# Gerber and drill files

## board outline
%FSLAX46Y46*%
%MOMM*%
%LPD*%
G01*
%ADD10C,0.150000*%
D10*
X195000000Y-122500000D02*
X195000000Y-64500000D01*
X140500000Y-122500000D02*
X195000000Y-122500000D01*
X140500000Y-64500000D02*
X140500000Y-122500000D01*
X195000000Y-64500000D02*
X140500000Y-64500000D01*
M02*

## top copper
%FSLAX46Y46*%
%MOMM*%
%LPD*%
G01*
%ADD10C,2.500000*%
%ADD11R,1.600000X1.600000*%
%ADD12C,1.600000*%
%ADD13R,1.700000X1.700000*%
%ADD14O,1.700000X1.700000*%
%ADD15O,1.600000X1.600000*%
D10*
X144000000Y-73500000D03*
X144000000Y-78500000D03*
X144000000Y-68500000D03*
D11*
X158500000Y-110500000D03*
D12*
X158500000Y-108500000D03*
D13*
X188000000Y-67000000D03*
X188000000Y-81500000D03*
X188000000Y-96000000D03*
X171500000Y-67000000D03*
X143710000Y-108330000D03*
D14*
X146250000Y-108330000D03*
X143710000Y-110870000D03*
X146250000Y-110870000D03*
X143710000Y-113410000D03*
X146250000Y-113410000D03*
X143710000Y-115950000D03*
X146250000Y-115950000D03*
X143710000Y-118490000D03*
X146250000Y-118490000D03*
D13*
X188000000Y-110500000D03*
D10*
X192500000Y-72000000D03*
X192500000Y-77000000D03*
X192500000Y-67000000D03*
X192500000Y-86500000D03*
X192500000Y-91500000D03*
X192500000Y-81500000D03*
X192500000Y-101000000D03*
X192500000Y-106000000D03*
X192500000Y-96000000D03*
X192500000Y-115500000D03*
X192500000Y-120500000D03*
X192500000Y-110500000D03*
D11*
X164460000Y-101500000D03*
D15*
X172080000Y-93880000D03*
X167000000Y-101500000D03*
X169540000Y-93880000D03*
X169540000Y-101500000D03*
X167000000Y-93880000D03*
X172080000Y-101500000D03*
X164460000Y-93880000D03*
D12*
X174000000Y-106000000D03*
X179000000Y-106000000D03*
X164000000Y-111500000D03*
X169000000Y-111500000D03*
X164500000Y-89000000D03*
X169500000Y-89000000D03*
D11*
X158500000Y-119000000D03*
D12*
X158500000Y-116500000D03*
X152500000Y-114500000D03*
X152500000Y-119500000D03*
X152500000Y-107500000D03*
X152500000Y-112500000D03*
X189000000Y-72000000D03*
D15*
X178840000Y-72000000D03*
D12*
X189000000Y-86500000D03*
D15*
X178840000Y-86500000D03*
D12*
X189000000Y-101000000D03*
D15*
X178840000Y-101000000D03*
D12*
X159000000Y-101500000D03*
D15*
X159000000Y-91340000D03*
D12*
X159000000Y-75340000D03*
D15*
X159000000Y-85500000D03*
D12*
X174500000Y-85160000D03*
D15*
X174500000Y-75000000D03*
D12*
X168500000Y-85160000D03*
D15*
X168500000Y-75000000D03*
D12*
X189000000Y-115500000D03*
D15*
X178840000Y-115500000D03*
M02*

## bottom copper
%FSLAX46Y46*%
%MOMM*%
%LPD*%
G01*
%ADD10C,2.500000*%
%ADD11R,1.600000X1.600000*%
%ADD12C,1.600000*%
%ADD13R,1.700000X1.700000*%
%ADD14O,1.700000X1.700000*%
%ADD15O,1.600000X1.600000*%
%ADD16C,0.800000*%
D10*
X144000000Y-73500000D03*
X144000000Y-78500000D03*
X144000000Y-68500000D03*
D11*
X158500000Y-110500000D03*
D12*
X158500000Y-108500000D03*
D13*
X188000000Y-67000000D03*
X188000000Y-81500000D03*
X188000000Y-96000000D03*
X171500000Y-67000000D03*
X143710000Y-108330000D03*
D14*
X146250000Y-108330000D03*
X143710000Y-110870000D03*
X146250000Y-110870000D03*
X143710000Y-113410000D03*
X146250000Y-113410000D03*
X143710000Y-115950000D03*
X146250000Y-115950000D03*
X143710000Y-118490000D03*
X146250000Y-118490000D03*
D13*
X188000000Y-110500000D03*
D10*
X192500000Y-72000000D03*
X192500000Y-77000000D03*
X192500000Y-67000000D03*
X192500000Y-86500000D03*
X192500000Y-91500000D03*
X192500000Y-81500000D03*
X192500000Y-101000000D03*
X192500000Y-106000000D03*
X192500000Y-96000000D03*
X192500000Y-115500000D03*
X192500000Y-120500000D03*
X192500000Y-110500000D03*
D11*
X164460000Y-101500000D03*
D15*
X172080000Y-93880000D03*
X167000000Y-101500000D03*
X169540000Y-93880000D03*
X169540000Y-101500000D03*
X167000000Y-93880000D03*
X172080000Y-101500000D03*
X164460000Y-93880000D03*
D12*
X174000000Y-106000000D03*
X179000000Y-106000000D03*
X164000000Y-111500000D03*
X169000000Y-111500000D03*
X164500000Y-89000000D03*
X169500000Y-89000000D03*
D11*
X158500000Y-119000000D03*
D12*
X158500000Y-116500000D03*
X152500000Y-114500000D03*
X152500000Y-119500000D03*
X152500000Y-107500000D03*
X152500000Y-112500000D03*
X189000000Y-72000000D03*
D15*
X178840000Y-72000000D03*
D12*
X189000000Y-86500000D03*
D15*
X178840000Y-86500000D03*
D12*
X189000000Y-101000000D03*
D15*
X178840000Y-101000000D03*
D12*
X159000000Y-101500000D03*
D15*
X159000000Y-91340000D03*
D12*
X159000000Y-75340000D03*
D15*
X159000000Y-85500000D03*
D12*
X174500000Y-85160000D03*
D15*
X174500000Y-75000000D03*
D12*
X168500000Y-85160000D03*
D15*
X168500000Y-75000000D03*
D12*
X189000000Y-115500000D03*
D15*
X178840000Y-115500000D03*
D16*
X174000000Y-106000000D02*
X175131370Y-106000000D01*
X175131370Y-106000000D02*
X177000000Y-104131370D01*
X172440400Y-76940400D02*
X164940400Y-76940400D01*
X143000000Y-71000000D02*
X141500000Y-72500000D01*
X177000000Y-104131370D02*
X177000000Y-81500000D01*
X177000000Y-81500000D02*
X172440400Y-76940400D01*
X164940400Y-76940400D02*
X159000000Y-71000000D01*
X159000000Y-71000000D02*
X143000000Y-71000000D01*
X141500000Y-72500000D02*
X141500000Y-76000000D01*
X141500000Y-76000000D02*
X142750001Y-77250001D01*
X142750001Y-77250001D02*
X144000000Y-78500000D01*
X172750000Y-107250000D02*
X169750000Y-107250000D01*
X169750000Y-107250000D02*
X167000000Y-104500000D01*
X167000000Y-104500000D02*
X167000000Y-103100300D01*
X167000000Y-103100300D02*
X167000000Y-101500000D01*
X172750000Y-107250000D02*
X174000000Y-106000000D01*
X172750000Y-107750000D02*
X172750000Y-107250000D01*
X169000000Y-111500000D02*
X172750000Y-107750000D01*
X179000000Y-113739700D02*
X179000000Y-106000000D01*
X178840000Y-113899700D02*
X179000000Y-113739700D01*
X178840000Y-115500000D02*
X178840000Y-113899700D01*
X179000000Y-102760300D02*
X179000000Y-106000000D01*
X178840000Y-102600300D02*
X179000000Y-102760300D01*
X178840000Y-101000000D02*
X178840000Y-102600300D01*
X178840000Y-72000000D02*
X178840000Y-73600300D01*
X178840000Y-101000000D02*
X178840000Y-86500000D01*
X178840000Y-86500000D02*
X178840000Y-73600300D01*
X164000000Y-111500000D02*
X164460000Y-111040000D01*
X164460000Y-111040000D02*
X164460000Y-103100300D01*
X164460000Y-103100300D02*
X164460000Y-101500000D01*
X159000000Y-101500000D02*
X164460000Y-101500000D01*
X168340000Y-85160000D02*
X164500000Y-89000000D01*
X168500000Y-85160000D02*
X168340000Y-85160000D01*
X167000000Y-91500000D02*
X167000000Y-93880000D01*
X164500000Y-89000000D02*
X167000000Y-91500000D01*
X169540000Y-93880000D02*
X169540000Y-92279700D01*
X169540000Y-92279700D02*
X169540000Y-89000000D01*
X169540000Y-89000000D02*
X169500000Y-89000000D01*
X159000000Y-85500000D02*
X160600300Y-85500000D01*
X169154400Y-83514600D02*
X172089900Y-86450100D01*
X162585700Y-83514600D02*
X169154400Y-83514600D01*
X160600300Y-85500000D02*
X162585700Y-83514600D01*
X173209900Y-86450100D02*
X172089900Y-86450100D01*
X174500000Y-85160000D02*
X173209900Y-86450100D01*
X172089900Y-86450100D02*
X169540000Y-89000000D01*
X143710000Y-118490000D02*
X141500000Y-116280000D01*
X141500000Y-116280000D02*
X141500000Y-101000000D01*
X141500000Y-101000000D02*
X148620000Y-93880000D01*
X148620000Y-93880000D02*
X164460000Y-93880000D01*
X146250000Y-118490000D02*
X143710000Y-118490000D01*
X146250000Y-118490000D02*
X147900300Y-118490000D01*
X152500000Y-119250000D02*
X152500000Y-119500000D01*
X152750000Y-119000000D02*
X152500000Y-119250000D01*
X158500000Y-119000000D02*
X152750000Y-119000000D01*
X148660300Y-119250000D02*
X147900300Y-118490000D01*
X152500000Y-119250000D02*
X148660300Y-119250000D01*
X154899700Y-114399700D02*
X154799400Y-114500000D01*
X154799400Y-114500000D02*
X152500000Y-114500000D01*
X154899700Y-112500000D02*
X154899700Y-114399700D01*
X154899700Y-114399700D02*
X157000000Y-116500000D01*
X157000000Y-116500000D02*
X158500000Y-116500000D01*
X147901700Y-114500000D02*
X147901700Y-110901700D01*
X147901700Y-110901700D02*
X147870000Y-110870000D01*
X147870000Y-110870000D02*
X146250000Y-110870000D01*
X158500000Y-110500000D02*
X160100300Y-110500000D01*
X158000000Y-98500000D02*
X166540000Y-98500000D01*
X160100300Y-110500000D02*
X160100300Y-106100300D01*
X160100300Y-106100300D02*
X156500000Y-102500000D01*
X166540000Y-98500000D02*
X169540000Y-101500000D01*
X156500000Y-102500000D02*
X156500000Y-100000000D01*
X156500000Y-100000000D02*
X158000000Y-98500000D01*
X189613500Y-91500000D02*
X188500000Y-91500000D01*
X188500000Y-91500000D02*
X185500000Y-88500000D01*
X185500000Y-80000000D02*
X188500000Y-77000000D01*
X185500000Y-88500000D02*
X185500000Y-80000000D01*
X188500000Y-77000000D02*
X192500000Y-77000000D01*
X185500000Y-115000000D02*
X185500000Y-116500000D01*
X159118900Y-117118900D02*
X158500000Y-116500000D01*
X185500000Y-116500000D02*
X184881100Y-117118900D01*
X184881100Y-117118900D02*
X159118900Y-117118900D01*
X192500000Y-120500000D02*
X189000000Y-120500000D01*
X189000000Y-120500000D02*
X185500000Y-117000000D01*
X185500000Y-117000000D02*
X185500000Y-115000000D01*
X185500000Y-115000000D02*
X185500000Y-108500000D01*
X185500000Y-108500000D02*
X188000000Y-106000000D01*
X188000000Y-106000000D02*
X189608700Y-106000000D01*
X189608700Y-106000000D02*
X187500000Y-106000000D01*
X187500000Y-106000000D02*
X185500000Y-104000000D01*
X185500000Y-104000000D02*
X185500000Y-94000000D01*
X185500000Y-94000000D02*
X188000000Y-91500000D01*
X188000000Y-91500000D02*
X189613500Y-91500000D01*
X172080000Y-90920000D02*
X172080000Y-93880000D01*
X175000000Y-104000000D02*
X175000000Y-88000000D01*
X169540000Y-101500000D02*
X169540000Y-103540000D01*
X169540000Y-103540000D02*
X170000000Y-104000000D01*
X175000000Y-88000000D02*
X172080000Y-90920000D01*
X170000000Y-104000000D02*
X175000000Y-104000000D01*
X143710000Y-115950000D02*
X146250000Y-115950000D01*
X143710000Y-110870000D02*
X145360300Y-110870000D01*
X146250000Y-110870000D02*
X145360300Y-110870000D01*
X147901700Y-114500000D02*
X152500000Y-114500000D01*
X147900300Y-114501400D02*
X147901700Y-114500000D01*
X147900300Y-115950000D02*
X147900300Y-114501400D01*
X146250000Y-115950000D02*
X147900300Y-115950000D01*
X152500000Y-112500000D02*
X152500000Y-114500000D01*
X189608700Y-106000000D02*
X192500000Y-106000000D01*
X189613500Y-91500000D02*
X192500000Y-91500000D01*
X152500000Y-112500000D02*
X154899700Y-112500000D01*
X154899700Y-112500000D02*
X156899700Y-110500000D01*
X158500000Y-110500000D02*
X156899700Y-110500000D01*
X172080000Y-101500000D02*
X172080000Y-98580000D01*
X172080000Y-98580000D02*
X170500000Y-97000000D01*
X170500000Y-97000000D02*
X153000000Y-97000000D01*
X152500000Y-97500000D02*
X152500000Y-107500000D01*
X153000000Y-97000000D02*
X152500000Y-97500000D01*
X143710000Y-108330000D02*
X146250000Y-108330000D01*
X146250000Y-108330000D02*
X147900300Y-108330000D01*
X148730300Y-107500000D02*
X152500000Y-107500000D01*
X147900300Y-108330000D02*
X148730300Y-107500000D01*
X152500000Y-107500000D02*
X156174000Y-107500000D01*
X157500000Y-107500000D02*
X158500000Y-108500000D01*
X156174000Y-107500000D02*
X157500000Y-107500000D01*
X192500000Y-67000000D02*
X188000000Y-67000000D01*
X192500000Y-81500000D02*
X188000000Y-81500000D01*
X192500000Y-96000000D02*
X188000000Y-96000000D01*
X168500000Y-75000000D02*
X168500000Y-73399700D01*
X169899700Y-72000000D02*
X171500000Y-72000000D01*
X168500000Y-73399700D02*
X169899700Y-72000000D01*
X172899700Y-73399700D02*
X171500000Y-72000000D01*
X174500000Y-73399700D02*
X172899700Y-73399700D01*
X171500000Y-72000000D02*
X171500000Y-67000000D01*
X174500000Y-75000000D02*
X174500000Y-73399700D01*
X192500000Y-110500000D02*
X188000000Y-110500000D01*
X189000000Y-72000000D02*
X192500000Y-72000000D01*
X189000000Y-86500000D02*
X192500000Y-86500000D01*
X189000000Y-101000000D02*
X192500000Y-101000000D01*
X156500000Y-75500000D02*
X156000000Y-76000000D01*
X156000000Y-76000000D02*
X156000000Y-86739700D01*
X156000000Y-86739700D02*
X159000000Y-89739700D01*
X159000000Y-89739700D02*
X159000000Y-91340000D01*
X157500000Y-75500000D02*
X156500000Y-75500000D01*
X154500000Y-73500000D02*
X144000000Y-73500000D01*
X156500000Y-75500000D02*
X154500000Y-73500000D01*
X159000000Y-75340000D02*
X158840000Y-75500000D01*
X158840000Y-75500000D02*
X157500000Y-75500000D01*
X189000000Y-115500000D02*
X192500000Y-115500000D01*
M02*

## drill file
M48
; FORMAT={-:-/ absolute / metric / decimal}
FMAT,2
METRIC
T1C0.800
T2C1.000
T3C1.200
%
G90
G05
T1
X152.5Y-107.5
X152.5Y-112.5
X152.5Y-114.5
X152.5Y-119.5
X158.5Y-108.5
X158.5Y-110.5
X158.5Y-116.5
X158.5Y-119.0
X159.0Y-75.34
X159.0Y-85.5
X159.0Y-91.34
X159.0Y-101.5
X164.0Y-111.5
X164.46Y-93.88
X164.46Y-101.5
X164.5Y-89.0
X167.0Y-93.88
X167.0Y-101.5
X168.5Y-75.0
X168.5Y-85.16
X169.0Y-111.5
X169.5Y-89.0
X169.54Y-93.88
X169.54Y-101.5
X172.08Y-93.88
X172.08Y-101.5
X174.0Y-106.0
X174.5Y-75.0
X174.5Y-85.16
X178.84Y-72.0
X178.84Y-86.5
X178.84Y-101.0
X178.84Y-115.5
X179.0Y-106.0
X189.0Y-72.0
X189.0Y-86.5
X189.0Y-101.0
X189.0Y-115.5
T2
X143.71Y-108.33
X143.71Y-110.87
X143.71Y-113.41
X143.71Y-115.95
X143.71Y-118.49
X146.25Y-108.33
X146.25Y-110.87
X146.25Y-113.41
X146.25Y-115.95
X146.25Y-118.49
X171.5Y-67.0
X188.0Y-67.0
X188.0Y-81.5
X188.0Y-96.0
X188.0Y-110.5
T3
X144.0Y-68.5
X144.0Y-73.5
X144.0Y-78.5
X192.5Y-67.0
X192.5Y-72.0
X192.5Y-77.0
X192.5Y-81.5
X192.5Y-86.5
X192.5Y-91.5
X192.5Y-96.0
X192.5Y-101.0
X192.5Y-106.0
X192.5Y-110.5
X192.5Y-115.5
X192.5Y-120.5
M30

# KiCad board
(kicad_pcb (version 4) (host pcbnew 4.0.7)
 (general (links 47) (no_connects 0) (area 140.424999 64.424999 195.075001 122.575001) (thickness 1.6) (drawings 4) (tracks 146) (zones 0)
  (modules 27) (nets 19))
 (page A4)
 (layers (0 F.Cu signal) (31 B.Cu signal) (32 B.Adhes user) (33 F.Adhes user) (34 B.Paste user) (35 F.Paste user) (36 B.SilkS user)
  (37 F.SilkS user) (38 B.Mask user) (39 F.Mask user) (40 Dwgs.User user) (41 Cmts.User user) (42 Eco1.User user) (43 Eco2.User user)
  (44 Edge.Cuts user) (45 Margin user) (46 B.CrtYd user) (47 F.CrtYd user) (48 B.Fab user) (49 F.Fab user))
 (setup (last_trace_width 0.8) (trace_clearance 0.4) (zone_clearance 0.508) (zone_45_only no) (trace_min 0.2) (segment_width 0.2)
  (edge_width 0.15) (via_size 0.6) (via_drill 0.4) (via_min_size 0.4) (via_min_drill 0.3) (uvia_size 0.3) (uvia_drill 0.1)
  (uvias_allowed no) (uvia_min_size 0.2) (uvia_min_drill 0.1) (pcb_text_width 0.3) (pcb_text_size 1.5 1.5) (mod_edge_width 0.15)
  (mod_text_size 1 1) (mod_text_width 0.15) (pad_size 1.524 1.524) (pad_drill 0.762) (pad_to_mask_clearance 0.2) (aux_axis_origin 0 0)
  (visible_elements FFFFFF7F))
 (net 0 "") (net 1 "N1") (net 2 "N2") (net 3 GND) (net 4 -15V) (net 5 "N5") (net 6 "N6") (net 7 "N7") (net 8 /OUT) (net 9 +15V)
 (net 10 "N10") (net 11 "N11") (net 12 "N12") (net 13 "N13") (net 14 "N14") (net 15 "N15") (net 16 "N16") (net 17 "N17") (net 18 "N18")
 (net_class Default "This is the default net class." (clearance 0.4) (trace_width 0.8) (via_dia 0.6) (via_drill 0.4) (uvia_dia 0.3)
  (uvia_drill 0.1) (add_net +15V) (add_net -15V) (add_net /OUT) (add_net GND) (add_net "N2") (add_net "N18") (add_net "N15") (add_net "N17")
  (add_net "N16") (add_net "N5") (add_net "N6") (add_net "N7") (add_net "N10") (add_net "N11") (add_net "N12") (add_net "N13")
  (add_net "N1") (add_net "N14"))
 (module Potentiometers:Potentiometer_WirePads (layer F.Cu) (at 144 68.5)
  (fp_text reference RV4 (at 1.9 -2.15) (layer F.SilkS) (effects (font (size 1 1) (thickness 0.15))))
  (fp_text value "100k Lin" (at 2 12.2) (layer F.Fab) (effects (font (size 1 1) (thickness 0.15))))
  (pad 2 thru_hole circle (at 0 5) (size 2.5 2.5) (drill 1.2) (layers *.Cu *.Mask) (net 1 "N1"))
  (pad 3 thru_hole circle (at 0 10) (size 2.5 2.5) (drill 1.2) (layers *.Cu *.Mask) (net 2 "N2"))
  (pad 1 thru_hole circle (at 0 0) (size 2.5 2.5) (drill 1.2) (layers *.Cu *.Mask)))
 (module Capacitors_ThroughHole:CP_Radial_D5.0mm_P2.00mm (layer F.Cu) (at 158.5 110.5 90)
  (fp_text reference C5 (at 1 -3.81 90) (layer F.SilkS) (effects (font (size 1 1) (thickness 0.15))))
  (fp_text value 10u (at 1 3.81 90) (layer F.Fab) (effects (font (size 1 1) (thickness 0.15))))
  (pad 1 thru_hole rect (at 0 0 90) (size 1.6 1.6) (drill 0.8) (layers *.Cu *.Mask) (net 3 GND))
  (pad 2 thru_hole circle (at 2 0 90) (size 1.6 1.6) (drill 0.8) (layers *.Cu *.Mask) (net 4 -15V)))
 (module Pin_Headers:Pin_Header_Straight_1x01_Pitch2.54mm (layer F.Cu) (at 188 67)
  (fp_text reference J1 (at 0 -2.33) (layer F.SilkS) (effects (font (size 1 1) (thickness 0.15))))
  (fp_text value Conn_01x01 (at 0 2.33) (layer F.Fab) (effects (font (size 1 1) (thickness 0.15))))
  (pad 1 thru_hole rect (at 0 0) (size 1.7 1.7) (drill 1) (layers *.Cu *.Mask) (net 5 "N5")))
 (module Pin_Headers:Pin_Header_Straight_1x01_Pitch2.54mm (layer F.Cu) (at 188 81.5)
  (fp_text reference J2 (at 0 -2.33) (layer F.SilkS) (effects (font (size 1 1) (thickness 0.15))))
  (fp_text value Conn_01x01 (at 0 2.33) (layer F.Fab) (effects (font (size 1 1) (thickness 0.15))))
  (pad 1 thru_hole rect (at 0 0) (size 1.7 1.7) (drill 1) (layers *.Cu *.Mask) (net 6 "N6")))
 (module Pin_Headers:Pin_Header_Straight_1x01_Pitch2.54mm (layer F.Cu) (at 188 96)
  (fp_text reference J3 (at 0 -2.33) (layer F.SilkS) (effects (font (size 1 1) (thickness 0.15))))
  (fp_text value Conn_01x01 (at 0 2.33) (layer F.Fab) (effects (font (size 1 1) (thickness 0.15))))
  (pad 1 thru_hole rect (at 0 0) (size 1.7 1.7) (drill 1) (layers *.Cu *.Mask) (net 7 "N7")))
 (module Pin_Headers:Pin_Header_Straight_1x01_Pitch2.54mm (layer F.Cu) (at 171.5 67)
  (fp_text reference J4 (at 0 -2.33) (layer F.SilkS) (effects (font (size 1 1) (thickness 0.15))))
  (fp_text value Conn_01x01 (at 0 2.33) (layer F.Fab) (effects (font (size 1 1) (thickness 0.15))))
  (pad 1 thru_hole rect (at 0 0) (size 1.7 1.7) (drill 1) (layers *.Cu *.Mask) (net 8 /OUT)))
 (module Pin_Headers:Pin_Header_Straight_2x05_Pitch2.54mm (layer F.Cu) (at 143.71 108.33)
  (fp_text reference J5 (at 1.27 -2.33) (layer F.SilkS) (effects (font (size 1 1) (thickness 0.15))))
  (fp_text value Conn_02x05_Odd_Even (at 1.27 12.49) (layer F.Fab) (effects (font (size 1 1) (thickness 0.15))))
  (pad 1 thru_hole rect (at 0 0) (size 1.7 1.7) (drill 1) (layers *.Cu *.Mask) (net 4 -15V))
  (pad 2 thru_hole oval (at 2.54 0) (size 1.7 1.7) (drill 1) (layers *.Cu *.Mask) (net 4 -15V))
  (pad 3 thru_hole oval (at 0 2.54) (size 1.7 1.7) (drill 1) (layers *.Cu *.Mask) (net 3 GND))
  (pad 4 thru_hole oval (at 2.54 2.54) (size 1.7 1.7) (drill 1) (layers *.Cu *.Mask) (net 3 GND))
  (pad 5 thru_hole oval (at 0 5.08) (size 1.7 1.7) (drill 1) (layers *.Cu *.Mask))
  (pad 6 thru_hole oval (at 2.54 5.08) (size 1.7 1.7) (drill 1) (layers *.Cu *.Mask))
  (pad 7 thru_hole oval (at 0 7.62) (size 1.7 1.7) (drill 1) (layers *.Cu *.Mask) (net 3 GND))
  (pad 8 thru_hole oval (at 2.54 7.62) (size 1.7 1.7) (drill 1) (layers *.Cu *.Mask) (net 3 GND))
  (pad 9 thru_hole oval (at 0 10.16) (size 1.7 1.7) (drill 1) (layers *.Cu *.Mask) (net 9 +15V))
  (pad 10 thru_hole oval (at 2.54 10.16) (size 1.7 1.7) (drill 1) (layers *.Cu *.Mask) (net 9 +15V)))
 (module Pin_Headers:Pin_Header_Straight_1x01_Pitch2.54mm (layer F.Cu) (at 188 110.5)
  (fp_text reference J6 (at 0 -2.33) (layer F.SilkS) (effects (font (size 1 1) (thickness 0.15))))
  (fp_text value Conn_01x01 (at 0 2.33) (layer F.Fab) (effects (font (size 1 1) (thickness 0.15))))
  (pad 1 thru_hole rect (at 0 0) (size 1.7 1.7) (drill 1) (layers *.Cu *.Mask) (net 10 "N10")))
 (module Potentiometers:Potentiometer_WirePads (layer F.Cu) (at 192.5 67)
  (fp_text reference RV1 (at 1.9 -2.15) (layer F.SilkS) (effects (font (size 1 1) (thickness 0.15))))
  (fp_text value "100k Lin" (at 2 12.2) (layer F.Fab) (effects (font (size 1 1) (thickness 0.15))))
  (pad 2 thru_hole circle (at 0 5) (size 2.5 2.5) (drill 1.2) (layers *.Cu *.Mask) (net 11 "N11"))
  (pad 3 thru_hole circle (at 0 10) (size 2.5 2.5) (drill 1.2) (layers *.Cu *.Mask) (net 3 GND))
  (pad 1 thru_hole circle (at 0 0) (size 2.5 2.5) (drill 1.2) (layers *.Cu *.Mask) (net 5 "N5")))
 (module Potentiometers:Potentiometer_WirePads (layer F.Cu) (at 192.5 81.5)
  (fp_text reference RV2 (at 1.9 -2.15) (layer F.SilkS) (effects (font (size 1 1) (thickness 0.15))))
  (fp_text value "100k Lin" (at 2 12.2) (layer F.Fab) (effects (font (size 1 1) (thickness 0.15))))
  (pad 2 thru_hole circle (at 0 5) (size 2.5 2.5) (drill 1.2) (layers *.Cu *.Mask) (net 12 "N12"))
  (pad 3 thru_hole circle (at 0 10) (size 2.5 2.5) (drill 1.2) (layers *.Cu *.Mask) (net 3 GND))
  (pad 1 thru_hole circle (at 0 0) (size 2.5 2.5) (drill 1.2) (layers *.Cu *.Mask) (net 6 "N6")))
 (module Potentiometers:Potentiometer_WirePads (layer F.Cu) (at 192.5 96)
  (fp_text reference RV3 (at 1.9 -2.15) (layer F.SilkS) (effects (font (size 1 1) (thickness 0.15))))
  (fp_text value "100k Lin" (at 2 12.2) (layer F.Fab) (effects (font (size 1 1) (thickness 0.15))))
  (pad 2 thru_hole circle (at 0 5) (size 2.5 2.5) (drill 1.2) (layers *.Cu *.Mask) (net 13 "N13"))
  (pad 3 thru_hole circle (at 0 10) (size 2.5 2.5) (drill 1.2) (layers *.Cu *.Mask) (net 3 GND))
  (pad 1 thru_hole circle (at 0 0) (size 2.5 2.5) (drill 1.2) (layers *.Cu *.Mask) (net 7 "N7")))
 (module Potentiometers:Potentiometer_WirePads (layer F.Cu) (at 192.5 110.5)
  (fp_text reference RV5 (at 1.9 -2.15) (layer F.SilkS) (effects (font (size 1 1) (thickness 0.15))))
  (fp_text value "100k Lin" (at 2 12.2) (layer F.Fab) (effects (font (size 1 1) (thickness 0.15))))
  (pad 2 thru_hole circle (at 0 5) (size 2.5 2.5) (drill 1.2) (layers *.Cu *.Mask) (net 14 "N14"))
  (pad 3 thru_hole circle (at 0 10) (size 2.5 2.5) (drill 1.2) (layers *.Cu *.Mask) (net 3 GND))
  (pad 1 thru_hole circle (at 0 0) (size 2.5 2.5) (drill 1.2) (layers *.Cu *.Mask) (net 10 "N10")))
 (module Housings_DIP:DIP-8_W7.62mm (layer F.Cu) (at 164.46 101.5 90)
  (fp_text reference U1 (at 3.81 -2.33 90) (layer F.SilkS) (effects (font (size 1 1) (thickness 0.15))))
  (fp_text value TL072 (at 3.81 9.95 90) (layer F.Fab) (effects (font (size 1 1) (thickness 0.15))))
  (pad 1 thru_hole rect (at 0 0 90) (size 1.6 1.6) (drill 0.8) (layers *.Cu *.Mask) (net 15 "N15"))
  (pad 5 thru_hole oval (at 7.62 7.62 90) (size 1.6 1.6) (drill 0.8) (layers *.Cu *.Mask) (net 3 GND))
  (pad 2 thru_hole oval (at 0 2.54 90) (size 1.6 1.6) (drill 0.8) (layers *.Cu *.Mask) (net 2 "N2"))
  (pad 6 thru_hole oval (at 7.62 5.08 90) (size 1.6 1.6) (drill 0.8) (layers *.Cu *.Mask) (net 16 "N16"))
  (pad 3 thru_hole oval (at 0 5.08 90) (size 1.6 1.6) (drill 0.8) (layers *.Cu *.Mask) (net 3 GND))
  (pad 7 thru_hole oval (at 7.62 2.54 90) (size 1.6 1.6) (drill 0.8) (layers *.Cu *.Mask) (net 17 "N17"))
  (pad 4 thru_hole oval (at 0 7.62 90) (size 1.6 1.6) (drill 0.8) (layers *.Cu *.Mask) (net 4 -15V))
  (pad 8 thru_hole oval (at 7.62 0 90) (size 1.6 1.6) (drill 0.8) (layers *.Cu *.Mask) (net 9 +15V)))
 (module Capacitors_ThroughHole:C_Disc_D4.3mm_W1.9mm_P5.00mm (layer F.Cu) (at 174 106)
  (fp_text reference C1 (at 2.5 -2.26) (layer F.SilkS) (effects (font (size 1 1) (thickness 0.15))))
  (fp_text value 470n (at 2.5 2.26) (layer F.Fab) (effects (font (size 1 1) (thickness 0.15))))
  (pad 1 thru_hole circle (at 0 0) (size 1.6 1.6) (drill 0.8) (layers *.Cu *.Mask) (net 2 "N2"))
  (pad 2 thru_hole circle (at 5 0) (size 1.6 1.6) (drill 0.8) (layers *.Cu *.Mask) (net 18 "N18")))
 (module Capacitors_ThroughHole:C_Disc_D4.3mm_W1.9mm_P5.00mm (layer F.Cu) (at 164 111.5)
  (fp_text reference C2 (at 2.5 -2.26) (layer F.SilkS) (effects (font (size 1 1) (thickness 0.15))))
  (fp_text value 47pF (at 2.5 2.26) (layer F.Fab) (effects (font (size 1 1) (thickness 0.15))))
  (pad 1 thru_hole circle (at 0 0) (size 1.6 1.6) (drill 0.8) (layers *.Cu *.Mask) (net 15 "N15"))
  (pad 2 thru_hole circle (at 5 0) (size 1.6 1.6) (drill 0.8) (layers *.Cu *.Mask) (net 2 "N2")))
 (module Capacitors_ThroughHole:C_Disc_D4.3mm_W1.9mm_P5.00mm (layer F.Cu) (at 164.5 89)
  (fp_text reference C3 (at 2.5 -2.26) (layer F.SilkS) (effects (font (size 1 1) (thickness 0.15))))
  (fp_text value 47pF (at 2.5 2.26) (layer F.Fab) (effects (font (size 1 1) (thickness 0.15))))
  (pad 1 thru_hole circle (at 0 0) (size 1.6 1.6) (drill 0.8) (layers *.Cu *.Mask) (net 17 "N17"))
  (pad 2 thru_hole circle (at 5 0) (size 1.6 1.6) (drill 0.8) (layers *.Cu *.Mask) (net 16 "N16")))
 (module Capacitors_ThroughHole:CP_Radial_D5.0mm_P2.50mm (layer F.Cu) (at 158.5 119 90)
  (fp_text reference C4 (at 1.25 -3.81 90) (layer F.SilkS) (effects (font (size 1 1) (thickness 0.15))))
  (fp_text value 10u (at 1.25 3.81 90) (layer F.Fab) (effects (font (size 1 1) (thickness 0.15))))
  (pad 1 thru_hole rect (at 0 0 90) (size 1.6 1.6) (drill 0.8) (layers *.Cu *.Mask) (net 9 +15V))
  (pad 2 thru_hole circle (at 2.5 0 90) (size 1.6 1.6) (drill 0.8) (layers *.Cu *.Mask) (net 3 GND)))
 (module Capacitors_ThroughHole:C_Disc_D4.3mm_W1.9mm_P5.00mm (layer F.Cu) (at 152.5 114.5 270)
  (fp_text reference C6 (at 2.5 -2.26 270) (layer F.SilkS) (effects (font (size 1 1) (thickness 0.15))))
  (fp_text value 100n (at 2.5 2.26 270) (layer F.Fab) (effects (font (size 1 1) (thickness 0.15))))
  (pad 1 thru_hole circle (at 0 0 270) (size 1.6 1.6) (drill 0.8) (layers *.Cu *.Mask) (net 3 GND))
  (pad 2 thru_hole circle (at 5 0 270) (size 1.6 1.6) (drill 0.8) (layers *.Cu *.Mask) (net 9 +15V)))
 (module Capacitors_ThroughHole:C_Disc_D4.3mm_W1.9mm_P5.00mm (layer F.Cu) (at 152.5 107.5 270)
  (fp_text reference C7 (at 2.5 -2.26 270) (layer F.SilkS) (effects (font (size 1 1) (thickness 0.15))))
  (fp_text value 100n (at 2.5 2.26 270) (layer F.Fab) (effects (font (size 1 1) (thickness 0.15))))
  (pad 1 thru_hole circle (at 0 0 270) (size 1.6 1.6) (drill 0.8) (layers *.Cu *.Mask) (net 4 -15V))
  (pad 2 thru_hole circle (at 5 0 270) (size 1.6 1.6) (drill 0.8) (layers *.Cu *.Mask) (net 3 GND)))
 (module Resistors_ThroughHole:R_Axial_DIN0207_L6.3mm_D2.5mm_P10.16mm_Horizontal (layer F.Cu) (at 189 72 180)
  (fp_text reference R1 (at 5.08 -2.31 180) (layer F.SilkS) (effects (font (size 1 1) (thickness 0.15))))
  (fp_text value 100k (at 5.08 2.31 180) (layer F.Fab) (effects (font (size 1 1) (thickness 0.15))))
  (pad 1 thru_hole circle (at 0 0 180) (size 1.6 1.6) (drill 0.8) (layers *.Cu *.Mask) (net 11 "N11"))
  (pad 2 thru_hole oval (at 10.16 0 180) (size 1.6 1.6) (drill 0.8) (layers *.Cu *.Mask) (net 18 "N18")))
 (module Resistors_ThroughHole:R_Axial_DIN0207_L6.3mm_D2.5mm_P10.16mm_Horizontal (layer F.Cu) (at 189 86.5 180)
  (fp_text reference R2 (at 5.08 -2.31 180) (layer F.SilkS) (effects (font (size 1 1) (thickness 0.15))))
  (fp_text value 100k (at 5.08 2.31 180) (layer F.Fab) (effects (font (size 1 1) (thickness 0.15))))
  (pad 1 thru_hole circle (at 0 0 180) (size 1.6 1.6) (drill 0.8) (layers *.Cu *.Mask) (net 12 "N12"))
  (pad 2 thru_hole oval (at 10.16 0 180) (size 1.6 1.6) (drill 0.8) (layers *.Cu *.Mask) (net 18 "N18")))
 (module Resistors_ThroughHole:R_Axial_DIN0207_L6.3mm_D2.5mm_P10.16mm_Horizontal (layer F.Cu) (at 189 101 180)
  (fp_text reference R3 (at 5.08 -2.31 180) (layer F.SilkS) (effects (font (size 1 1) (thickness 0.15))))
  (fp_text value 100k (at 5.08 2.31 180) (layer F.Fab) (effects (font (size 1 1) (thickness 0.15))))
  (pad 1 thru_hole circle (at 0 0 180) (size 1.6 1.6) (drill 0.8) (layers *.Cu *.Mask) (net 13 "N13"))
  (pad 2 thru_hole oval (at 10.16 0 180) (size 1.6 1.6) (drill 0.8) (layers *.Cu *.Mask) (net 18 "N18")))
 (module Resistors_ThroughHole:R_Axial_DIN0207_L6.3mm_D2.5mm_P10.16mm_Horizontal (layer F.Cu) (at 159 101.5 90)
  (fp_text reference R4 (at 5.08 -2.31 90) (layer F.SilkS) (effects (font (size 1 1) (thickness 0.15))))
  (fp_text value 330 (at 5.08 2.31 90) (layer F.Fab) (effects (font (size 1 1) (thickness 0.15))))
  (pad 1 thru_hole circle (at 0 0 90) (size 1.6 1.6) (drill 0.8) (layers *.Cu *.Mask) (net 15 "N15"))
  (pad 2 thru_hole oval (at 10.16 0 90) (size 1.6 1.6) (drill 0.8) (layers *.Cu *.Mask) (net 1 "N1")))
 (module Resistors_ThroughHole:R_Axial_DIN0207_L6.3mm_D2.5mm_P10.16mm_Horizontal (layer F.Cu) (at 159 75.34 270)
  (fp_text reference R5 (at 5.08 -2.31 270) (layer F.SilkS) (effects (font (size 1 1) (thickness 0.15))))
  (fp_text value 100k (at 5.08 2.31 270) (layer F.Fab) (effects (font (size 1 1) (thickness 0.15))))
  (pad 1 thru_hole circle (at 0 0 270) (size 1.6 1.6) (drill 0.8) (layers *.Cu *.Mask) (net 1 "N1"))
  (pad 2 thru_hole oval (at 10.16 0 270) (size 1.6 1.6) (drill 0.8) (layers *.Cu *.Mask) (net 16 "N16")))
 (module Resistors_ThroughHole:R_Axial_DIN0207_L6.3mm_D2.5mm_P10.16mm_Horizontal (layer F.Cu) (at 174.5 85.16 90)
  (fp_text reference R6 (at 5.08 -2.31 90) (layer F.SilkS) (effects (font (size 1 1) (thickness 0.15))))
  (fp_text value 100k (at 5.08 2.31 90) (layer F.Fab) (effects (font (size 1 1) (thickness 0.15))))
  (pad 1 thru_hole circle (at 0 0 90) (size 1.6 1.6) (drill 0.8) (layers *.Cu *.Mask) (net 16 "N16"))
  (pad 2 thru_hole oval (at 10.16 0 90) (size 1.6 1.6) (drill 0.8) (layers *.Cu *.Mask) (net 8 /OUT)))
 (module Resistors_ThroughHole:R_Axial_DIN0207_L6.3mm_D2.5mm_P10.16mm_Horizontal (layer F.Cu) (at 168.5 85.16 90)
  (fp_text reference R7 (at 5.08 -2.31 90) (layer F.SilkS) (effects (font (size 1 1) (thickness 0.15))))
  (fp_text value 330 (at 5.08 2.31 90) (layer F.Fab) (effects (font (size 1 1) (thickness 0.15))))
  (pad 1 thru_hole circle (at 0 0 90) (size 1.6 1.6) (drill 0.8) (layers *.Cu *.Mask) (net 17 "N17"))
  (pad 2 thru_hole oval (at 10.16 0 90) (size 1.6 1.6) (drill 0.8) (layers *.Cu *.Mask) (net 8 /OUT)))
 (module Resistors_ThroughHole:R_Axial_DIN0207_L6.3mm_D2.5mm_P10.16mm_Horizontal (layer F.Cu) (at 189 115.5 180)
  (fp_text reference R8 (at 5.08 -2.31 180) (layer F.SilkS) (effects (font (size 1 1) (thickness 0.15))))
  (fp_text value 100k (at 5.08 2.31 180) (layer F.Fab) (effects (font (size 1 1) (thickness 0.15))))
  (pad 1 thru_hole circle (at 0 0 180) (size 1.6 1.6) (drill 0.8) (layers *.Cu *.Mask) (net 14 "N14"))
  (pad 2 thru_hole oval (at 10.16 0 180) (size 1.6 1.6) (drill 0.8) (layers *.Cu *.Mask) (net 18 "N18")))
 (gr_line (start 195 122.5) (end 195 64.5) (angle 90) (layer Edge.Cuts) (width 0.15))
 (gr_line (start 140.5 122.5) (end 195 122.5) (angle 90) (layer Edge.Cuts) (width 0.15))
 (gr_line (start 140.5 64.5) (end 140.5 122.5) (angle 90) (layer Edge.Cuts) (width 0.15))
 (gr_line (start 195 64.5) (end 140.5 64.5) (angle 90) (layer Edge.Cuts) (width 0.15))
 (segment (start 174 106) (end 175.13137 106) (width 0.8) (layer B.Cu) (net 2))
 (segment (start 175.13137 106) (end 177 104.13137) (width 0.8) (layer B.Cu) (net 2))
 (segment (start 172.4404 76.9404) (end 164.9404 76.9404) (width 0.8) (layer B.Cu) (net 2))
 (segment (start 143 71) (end 141.5 72.5) (width 0.8) (layer B.Cu) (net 2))
 (segment (start 177 104.13137) (end 177 81.5) (width 0.8) (layer B.Cu) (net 2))
 (segment (start 177 81.5) (end 172.4404 76.9404) (width 0.8) (layer B.Cu) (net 2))
 (segment (start 164.9404 76.9404) (end 159 71) (width 0.8) (layer B.Cu) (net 2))
 (segment (start 159 71) (end 143 71) (width 0.8) (layer B.Cu) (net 2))
 (segment (start 141.5 72.5) (end 141.5 76) (width 0.8) (layer B.Cu) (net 2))
 (segment (start 141.5 76) (end 142.750001 77.250001) (width 0.8) (layer B.Cu) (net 2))
 (segment (start 142.750001 77.250001) (end 144 78.5) (width 0.8) (layer B.Cu) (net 2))
 (segment (start 172.75 107.25) (end 169.75 107.25) (width 0.8) (layer B.Cu) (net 2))
 (segment (start 169.75 107.25) (end 167 104.5) (width 0.8) (layer B.Cu) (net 2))
 (segment (start 167 104.5) (end 167 103.1003) (width 0.8) (layer B.Cu) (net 2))
 (segment (start 167 103.1003) (end 167 101.5) (width 0.8) (layer B.Cu) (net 2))
 (segment (start 172.75 107.25) (end 174 106) (width 0.8) (layer B.Cu) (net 2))
 (segment (start 172.75 107.75) (end 172.75 107.25) (width 0.8) (layer B.Cu) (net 2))
 (segment (start 169 111.5) (end 172.75 107.75) (width 0.8) (layer B.Cu) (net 2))
 (segment (start 179 113.7397) (end 179 106) (width 0.8) (layer B.Cu) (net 18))
 (segment (start 178.84 113.8997) (end 179 113.7397) (width 0.8) (layer B.Cu) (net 18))
 (segment (start 178.84 115.5) (end 178.84 113.8997) (width 0.8) (layer B.Cu) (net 18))
 (segment (start 179 102.7603) (end 179 106) (width 0.8) (layer B.Cu) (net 18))
 (segment (start 178.84 102.6003) (end 179 102.7603) (width 0.8) (layer B.Cu) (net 18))
 (segment (start 178.84 101) (end 178.84 102.6003) (width 0.8) (layer B.Cu) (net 18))
 (segment (start 178.84 72) (end 178.84 73.6003) (width 0.8) (layer B.Cu) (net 18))
 (segment (start 178.84 101) (end 178.84 86.5) (width 0.8) (layer B.Cu) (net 18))
 (segment (start 178.84 86.5) (end 178.84 73.6003) (width 0.8) (layer B.Cu) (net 18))
 (segment (start 164 111.5) (end 164.46 111.04) (width 0.8) (layer B.Cu) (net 15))
 (segment (start 164.46 111.04) (end 164.46 103.1003) (width 0.8) (layer B.Cu) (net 15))
 (segment (start 164.46 103.1003) (end 164.46 101.5) (width 0.8) (layer B.Cu) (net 15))
 (segment (start 159 101.5) (end 164.46 101.5) (width 0.8) (layer B.Cu) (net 15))
 (segment (start 168.34 85.16) (end 164.5 89) (width 0.8) (layer B.Cu) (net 17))
 (segment (start 168.5 85.16) (end 168.34 85.16) (width 0.8) (layer B.Cu) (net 17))
 (segment (start 167 91.5) (end 167 93.88) (width 0.8) (layer B.Cu) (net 17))
 (segment (start 164.5 89) (end 167 91.5) (width 0.8) (layer B.Cu) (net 17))
 (segment (start 169.54 93.88) (end 169.54 92.2797) (width 0.8) (layer B.Cu) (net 16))
 (segment (start 169.54 92.2797) (end 169.54 89) (width 0.8) (layer B.Cu) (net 16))
 (segment (start 169.54 89) (end 169.5 89) (width 0.8) (layer B.Cu) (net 16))
 (segment (start 159 85.5) (end 160.6003 85.5) (width 0.8) (layer B.Cu) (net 16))
 (segment (start 169.1544 83.5146) (end 172.0899 86.4501) (width 0.8) (layer B.Cu) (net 16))
 (segment (start 162.5857 83.5146) (end 169.1544 83.5146) (width 0.8) (layer B.Cu) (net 16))
 (segment (start 160.6003 85.5) (end 162.5857 83.5146) (width 0.8) (layer B.Cu) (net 16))
 (segment (start 173.2099 86.4501) (end 172.0899 86.4501) (width 0.8) (layer B.Cu) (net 16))
 (segment (start 174.5 85.16) (end 173.2099 86.4501) (width 0.8) (layer B.Cu) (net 16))
 (segment (start 172.0899 86.4501) (end 169.54 89) (width 0.8) (layer B.Cu) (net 16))
 (segment (start 143.71 118.49) (end 141.5 116.28) (width 0.8) (layer B.Cu) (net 9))
 (segment (start 141.5 116.28) (end 141.5 101) (width 0.8) (layer B.Cu) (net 9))
 (segment (start 141.5 101) (end 148.62 93.88) (width 0.8) (layer B.Cu) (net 9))
 (segment (start 148.62 93.88) (end 164.46 93.88) (width 0.8) (layer B.Cu) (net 9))
 (segment (start 146.25 118.49) (end 143.71 118.49) (width 0.8) (layer B.Cu) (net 9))
 (segment (start 146.25 118.49) (end 147.9003 118.49) (width 0.8) (layer B.Cu) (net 9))
 (segment (start 152.5 119.25) (end 152.5 119.5) (width 0.8) (layer B.Cu) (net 9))
 (segment (start 152.75 119) (end 152.5 119.25) (width 0.8) (layer B.Cu) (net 9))
 (segment (start 158.5 119) (end 152.75 119) (width 0.8) (layer B.Cu) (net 9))
 (segment (start 148.6603 119.25) (end 147.9003 118.49) (width 0.8) (layer B.Cu) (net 9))
 (segment (start 152.5 119.25) (end 148.6603 119.25) (width 0.8) (layer B.Cu) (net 9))
 (segment (start 154.8997 114.3997) (end 154.7994 114.5) (width 0.8) (layer B.Cu) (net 3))
 (segment (start 154.7994 114.5) (end 152.5 114.5) (width 0.8) (layer B.Cu) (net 3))
 (segment (start 154.8997 112.5) (end 154.8997 114.3997) (width 0.8) (layer B.Cu) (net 3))
 (segment (start 154.8997 114.3997) (end 157 116.5) (width 0.8) (layer B.Cu) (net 3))
 (segment (start 157 116.5) (end 158.5 116.5) (width 0.8) (layer B.Cu) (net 3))
 (segment (start 147.9017 114.5) (end 147.9017 110.9017) (width 0.8) (layer B.Cu) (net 3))
 (segment (start 147.9017 110.9017) (end 147.87 110.87) (width 0.8) (layer B.Cu) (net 3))
 (segment (start 147.87 110.87) (end 146.25 110.87) (width 0.8) (layer B.Cu) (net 3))
 (segment (start 158.5 110.5) (end 160.1003 110.5) (width 0.8) (layer B.Cu) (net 3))
 (segment (start 158 98.5) (end 166.54 98.5) (width 0.8) (layer B.Cu) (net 3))
 (segment (start 160.1003 110.5) (end 160.1003 106.1003) (width 0.8) (layer B.Cu) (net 3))
 (segment (start 160.1003 106.1003) (end 156.5 102.5) (width 0.8) (layer B.Cu) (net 3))
 (segment (start 166.54 98.5) (end 169.54 101.5) (width 0.8) (layer B.Cu) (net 3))
 (segment (start 156.5 102.5) (end 156.5 100) (width 0.8) (layer B.Cu) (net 3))
 (segment (start 156.5 100) (end 158 98.5) (width 0.8) (layer B.Cu) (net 3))
 (segment (start 189.6135 91.5) (end 188.5 91.5) (width 0.8) (layer B.Cu) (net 3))
 (segment (start 188.5 91.5) (end 185.5 88.5) (width 0.8) (layer B.Cu) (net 3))
 (segment (start 185.5 80) (end 188.5 77) (width 0.8) (layer B.Cu) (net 3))
 (segment (start 185.5 88.5) (end 185.5 80) (width 0.8) (layer B.Cu) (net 3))
 (segment (start 188.5 77) (end 192.5 77) (width 0.8) (layer B.Cu) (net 3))
 (segment (start 185.5 115) (end 185.5 116.5) (width 0.8) (layer B.Cu) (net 3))
 (segment (start 159.1189 117.1189) (end 158.5 116.5) (width 0.8) (layer B.Cu) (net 3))
 (segment (start 185.5 116.5) (end 184.8811 117.1189) (width 0.8) (layer B.Cu) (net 3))
 (segment (start 184.8811 117.1189) (end 159.1189 117.1189) (width 0.8) (layer B.Cu) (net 3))
 (segment (start 192.5 120.5) (end 189 120.5) (width 0.8) (layer B.Cu) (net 3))
 (segment (start 189 120.5) (end 185.5 117) (width 0.8) (layer B.Cu) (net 3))
 (segment (start 185.5 117) (end 185.5 115) (width 0.8) (layer B.Cu) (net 3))
 (segment (start 185.5 115) (end 185.5 108.5) (width 0.8) (layer B.Cu) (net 3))
 (segment (start 185.5 108.5) (end 188 106) (width 0.8) (layer B.Cu) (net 3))
 (segment (start 188 106) (end 189.6087 106) (width 0.8) (layer B.Cu) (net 3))
 (segment (start 189.6087 106) (end 187.5 106) (width 0.8) (layer B.Cu) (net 3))
 (segment (start 187.5 106) (end 185.5 104) (width 0.8) (layer B.Cu) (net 3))
 (segment (start 185.5 104) (end 185.5 94) (width 0.8) (layer B.Cu) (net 3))
 (segment (start 185.5 94) (end 188 91.5) (width 0.8) (layer B.Cu) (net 3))
 (segment (start 188 91.5) (end 189.6135 91.5) (width 0.8) (layer B.Cu) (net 3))
 (segment (start 172.08 90.92) (end 172.08 93.88) (width 0.8) (layer B.Cu) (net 3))
 (segment (start 175 104) (end 175 88) (width 0.8) (layer B.Cu) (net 3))
 (segment (start 169.54 101.5) (end 169.54 103.54) (width 0.8) (layer B.Cu) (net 3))
 (segment (start 169.54 103.54) (end 170 104) (width 0.8) (layer B.Cu) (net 3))
 (segment (start 175 88) (end 172.08 90.92) (width 0.8) (layer B.Cu) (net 3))
 (segment (start 170 104) (end 175 104) (width 0.8) (layer B.Cu) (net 3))
 (segment (start 143.71 115.95) (end 146.25 115.95) (width 0.8) (layer B.Cu) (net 3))
 (segment (start 143.71 110.87) (end 145.3603 110.87) (width 0.8) (layer B.Cu) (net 3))
 (segment (start 146.25 110.87) (end 145.3603 110.87) (width 0.8) (layer B.Cu) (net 3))
 (segment (start 147.9017 114.5) (end 152.5 114.5) (width 0.8) (layer B.Cu) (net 3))
 (segment (start 147.9003 114.5014) (end 147.9017 114.5) (width 0.8) (layer B.Cu) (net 3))
 (segment (start 147.9003 115.95) (end 147.9003 114.5014) (width 0.8) (layer B.Cu) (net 3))
 (segment (start 146.25 115.95) (end 147.9003 115.95) (width 0.8) (layer B.Cu) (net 3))
 (segment (start 152.5 112.5) (end 152.5 114.5) (width 0.8) (layer B.Cu) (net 3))
 (segment (start 189.6087 106) (end 192.5 106) (width 0.8) (layer B.Cu) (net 3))
 (segment (start 189.6135 91.5) (end 192.5 91.5) (width 0.8) (layer B.Cu) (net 3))
 (segment (start 152.5 112.5) (end 154.8997 112.5) (width 0.8) (layer B.Cu) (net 3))
 (segment (start 154.8997 112.5) (end 156.8997 110.5) (width 0.8) (layer B.Cu) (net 3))
 (segment (start 158.5 110.5) (end 156.8997 110.5) (width 0.8) (layer B.Cu) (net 3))
 (segment (start 172.08 101.5) (end 172.08 98.58) (width 0.8) (layer B.Cu) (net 4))
 (segment (start 172.08 98.58) (end 170.5 97) (width 0.8) (layer B.Cu) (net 4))
 (segment (start 170.5 97) (end 153 97) (width 0.8) (layer B.Cu) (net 4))
 (segment (start 152.5 97.5) (end 152.5 107.5) (width 0.8) (layer B.Cu) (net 4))
 (segment (start 153 97) (end 152.5 97.5) (width 0.8) (layer B.Cu) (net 4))
 (segment (start 143.71 108.33) (end 146.25 108.33) (width 0.8) (layer B.Cu) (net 4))
 (segment (start 146.25 108.33) (end 147.9003 108.33) (width 0.8) (layer B.Cu) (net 4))
 (segment (start 148.7303 107.5) (end 152.5 107.5) (width 0.8) (layer B.Cu) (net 4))
 (segment (start 147.9003 108.33) (end 148.7303 107.5) (width 0.8) (layer B.Cu) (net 4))
 (segment (start 152.5 107.5) (end 156.174 107.5) (width 0.8) (layer B.Cu) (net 4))
 (segment (start 157.5 107.5) (end 158.5 108.5) (width 0.8) (layer B.Cu) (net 4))
 (segment (start 156.174 107.5) (end 157.5 107.5) (width 0.8) (layer B.Cu) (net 4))
 (segment (start 192.5 67) (end 188 67) (width 0.8) (layer B.Cu) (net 5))
 (segment (start 192.5 81.5) (end 188 81.5) (width 0.8) (layer B.Cu) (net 6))
 (segment (start 192.5 96) (end 188 96) (width 0.8) (layer B.Cu) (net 7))
 (segment (start 168.5 75) (end 168.5 73.3997) (width 0.8) (layer B.Cu) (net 8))
 (segment (start 169.8997 72) (end 171.5 72) (width 0.8) (layer B.Cu) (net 8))
 (segment (start 168.5 73.3997) (end 169.8997 72) (width 0.8) (layer B.Cu) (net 8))
 (segment (start 172.8997 73.3997) (end 171.5 72) (width 0.8) (layer B.Cu) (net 8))
 (segment (start 174.5 73.3997) (end 172.8997 73.3997) (width 0.8) (layer B.Cu) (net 8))
 (segment (start 171.5 72) (end 171.5 67) (width 0.8) (layer B.Cu) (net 8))
 (segment (start 174.5 75) (end 174.5 73.3997) (width 0.8) (layer B.Cu) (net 8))
 (segment (start 192.5 110.5) (end 188 110.5) (width 0.8) (layer B.Cu) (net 10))
 (segment (start 189 72) (end 192.5 72) (width 0.8) (layer B.Cu) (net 11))
 (segment (start 189 86.5) (end 192.5 86.5) (width 0.8) (layer B.Cu) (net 12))
 (segment (start 189 101) (end 192.5 101) (width 0.8) (layer B.Cu) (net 13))
 (segment (start 156.5 75.5) (end 156 76) (width 0.8) (layer B.Cu) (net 1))
 (segment (start 156 76) (end 156 86.7397) (width 0.8) (layer B.Cu) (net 1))
 (segment (start 156 86.7397) (end 159 89.7397) (width 0.8) (layer B.Cu) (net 1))
 (segment (start 159 89.7397) (end 159 91.34) (width 0.8) (layer B.Cu) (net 1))
 (segment (start 157.5 75.5) (end 156.5 75.5) (width 0.8) (layer B.Cu) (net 1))
 (segment (start 154.5 73.5) (end 144 73.5) (width 0.8) (layer B.Cu) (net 1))
 (segment (start 156.5 75.5) (end 154.5 73.5) (width 0.8) (layer B.Cu) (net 1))
 (segment (start 159 75.34) (end 158.84 75.5) (width 0.8) (layer B.Cu) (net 1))
 (segment (start 158.84 75.5) (end 157.5 75.5) (width 0.8) (layer B.Cu) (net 1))
 (segment (start 189 115.5) (end 192.5 115.5) (width 0.8) (layer B.Cu) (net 14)))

